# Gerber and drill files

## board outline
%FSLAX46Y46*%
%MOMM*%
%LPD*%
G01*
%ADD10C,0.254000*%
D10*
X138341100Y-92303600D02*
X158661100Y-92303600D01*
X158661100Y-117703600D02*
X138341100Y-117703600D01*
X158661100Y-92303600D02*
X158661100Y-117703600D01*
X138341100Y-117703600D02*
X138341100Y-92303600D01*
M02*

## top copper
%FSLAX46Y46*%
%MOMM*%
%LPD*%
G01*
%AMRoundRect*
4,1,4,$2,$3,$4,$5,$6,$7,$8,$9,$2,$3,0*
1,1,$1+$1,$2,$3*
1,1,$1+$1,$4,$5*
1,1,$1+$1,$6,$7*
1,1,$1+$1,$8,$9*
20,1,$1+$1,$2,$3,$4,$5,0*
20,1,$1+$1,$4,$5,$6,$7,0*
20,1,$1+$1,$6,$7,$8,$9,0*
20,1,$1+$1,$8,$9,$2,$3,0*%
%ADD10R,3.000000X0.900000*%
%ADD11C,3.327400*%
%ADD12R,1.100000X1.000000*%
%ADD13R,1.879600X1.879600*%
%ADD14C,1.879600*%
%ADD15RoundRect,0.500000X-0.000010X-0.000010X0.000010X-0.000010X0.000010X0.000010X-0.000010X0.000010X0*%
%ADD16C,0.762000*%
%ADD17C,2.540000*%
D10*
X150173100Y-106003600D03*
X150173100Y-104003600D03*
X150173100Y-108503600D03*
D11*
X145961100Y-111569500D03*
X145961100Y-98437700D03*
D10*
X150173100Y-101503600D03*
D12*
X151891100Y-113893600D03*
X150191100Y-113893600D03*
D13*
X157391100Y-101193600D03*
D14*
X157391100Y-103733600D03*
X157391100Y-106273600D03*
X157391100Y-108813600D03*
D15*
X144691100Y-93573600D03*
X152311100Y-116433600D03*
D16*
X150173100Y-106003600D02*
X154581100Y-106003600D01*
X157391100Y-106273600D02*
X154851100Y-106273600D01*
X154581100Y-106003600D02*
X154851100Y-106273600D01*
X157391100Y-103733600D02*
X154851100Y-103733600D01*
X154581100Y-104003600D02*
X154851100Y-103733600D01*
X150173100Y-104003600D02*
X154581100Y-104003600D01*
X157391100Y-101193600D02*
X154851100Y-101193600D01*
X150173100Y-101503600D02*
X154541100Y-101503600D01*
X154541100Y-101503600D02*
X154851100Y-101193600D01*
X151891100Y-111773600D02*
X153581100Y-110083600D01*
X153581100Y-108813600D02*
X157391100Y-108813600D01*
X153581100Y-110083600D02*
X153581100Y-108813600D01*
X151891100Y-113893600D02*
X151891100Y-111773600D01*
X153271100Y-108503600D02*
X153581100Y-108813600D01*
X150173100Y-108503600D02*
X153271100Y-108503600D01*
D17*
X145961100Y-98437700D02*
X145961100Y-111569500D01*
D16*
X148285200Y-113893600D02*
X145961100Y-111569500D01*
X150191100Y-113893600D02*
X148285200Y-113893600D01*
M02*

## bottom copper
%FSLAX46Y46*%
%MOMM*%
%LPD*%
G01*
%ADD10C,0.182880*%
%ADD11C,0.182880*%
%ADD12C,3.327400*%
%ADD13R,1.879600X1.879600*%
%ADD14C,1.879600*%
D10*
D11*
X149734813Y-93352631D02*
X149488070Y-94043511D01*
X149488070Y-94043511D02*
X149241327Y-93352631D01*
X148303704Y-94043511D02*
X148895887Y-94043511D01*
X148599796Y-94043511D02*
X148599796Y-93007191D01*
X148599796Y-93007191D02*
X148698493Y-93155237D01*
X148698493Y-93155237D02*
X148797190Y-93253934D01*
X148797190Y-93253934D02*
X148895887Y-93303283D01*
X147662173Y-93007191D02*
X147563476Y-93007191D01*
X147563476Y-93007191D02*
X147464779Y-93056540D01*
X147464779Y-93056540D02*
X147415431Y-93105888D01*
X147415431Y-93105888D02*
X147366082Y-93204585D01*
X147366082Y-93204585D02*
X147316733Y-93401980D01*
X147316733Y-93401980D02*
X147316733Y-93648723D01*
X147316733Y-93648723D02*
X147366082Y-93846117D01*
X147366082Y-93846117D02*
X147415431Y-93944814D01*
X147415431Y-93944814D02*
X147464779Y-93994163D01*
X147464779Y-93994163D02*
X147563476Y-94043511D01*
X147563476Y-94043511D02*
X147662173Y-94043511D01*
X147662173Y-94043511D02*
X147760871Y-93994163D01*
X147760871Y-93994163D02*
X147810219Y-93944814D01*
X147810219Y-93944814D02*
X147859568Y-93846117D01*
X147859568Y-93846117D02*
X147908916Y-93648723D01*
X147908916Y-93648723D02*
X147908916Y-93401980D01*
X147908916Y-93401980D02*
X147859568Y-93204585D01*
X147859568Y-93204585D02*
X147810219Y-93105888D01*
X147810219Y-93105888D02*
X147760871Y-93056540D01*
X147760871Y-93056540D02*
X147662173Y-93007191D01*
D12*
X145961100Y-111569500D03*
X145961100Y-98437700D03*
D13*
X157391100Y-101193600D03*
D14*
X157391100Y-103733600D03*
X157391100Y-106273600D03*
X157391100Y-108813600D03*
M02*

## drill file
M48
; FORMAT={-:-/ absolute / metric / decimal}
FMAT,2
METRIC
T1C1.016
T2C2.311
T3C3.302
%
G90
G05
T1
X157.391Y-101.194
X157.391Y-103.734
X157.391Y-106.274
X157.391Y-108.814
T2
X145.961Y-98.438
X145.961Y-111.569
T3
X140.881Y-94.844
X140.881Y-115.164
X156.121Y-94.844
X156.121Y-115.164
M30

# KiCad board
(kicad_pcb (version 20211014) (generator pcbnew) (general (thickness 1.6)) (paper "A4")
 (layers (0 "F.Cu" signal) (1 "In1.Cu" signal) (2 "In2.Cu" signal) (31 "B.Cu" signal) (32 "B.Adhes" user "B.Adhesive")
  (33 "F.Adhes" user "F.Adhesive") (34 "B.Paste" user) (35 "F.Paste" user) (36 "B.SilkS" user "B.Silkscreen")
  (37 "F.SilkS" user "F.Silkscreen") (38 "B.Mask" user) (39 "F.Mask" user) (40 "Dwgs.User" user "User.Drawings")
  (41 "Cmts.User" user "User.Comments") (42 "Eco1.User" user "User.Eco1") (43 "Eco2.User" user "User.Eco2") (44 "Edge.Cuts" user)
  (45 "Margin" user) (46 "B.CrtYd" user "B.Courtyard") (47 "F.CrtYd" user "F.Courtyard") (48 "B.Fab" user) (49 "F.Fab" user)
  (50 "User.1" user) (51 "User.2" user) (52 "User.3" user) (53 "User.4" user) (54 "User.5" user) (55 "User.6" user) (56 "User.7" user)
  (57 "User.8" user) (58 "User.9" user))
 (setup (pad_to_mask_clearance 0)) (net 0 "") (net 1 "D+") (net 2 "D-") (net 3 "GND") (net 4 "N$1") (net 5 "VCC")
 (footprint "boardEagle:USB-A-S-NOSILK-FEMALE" (layer "F.Cu") (at 145.9611 105.0036)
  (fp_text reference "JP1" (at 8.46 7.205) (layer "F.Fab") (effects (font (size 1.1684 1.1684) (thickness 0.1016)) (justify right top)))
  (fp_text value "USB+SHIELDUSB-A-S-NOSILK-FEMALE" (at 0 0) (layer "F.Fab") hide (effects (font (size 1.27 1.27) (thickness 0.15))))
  (pad "D+" smd rect (at 4.212 1) (size 3 0.9) (layers "F.Cu" "F.Paste" "F.Mask") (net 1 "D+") (solder_mask_margin 0.1016))
  (pad "D-" smd rect (at 4.212 -1) (size 3 0.9) (layers "F.Cu" "F.Paste" "F.Mask") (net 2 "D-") (solder_mask_margin 0.1016))
  (pad "GND" smd rect (at 4.212 3.5) (size 3 0.9) (layers "F.Cu" "F.Paste" "F.Mask") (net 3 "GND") (solder_mask_margin 0.1016))
  (pad "S1" thru_hole circle (at 0 6.5659 270) (size 3.3274 3.3274) (drill 2.3114) (layers *.Cu *.Mask) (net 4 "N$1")
   (solder_mask_margin 0.1016))
  (pad "S2" thru_hole circle (at 0 -6.5659 270) (size 3.3274 3.3274) (drill 2.3114) (layers *.Cu *.Mask) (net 4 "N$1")
   (solder_mask_margin 0.1016))
  (pad "VBUS" smd rect (at 4.212 -3.5) (size 3 0.9) (layers "F.Cu" "F.Paste" "F.Mask") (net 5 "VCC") (solder_mask_margin 0.1016)))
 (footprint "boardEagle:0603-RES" (layer "F.Cu") (at 151.0411 113.8936 180)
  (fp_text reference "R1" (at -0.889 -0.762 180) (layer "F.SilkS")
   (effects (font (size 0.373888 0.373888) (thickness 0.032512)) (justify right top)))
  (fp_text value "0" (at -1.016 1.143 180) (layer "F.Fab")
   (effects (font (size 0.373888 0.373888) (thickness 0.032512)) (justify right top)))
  (pad "1" smd rect (at -0.85 0 180) (size 1.1 1) (layers "F.Cu" "F.Paste" "F.Mask") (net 3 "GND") (solder_mask_margin 0.1016))
  (pad "2" smd rect (at 0.85 0 180) (size 1.1 1) (layers "F.Cu" "F.Paste" "F.Mask") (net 4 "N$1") (solder_mask_margin 0.1016)))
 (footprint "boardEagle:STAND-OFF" (layer "F.Cu") (at 140.8811 94.8436)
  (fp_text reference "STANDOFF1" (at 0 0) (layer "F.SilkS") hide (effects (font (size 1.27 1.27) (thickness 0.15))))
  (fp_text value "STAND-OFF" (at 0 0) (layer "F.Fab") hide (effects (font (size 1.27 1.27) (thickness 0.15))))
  (pad "" np_thru_hole circle (at 0 0) (size 3.302 3.302) (drill 3.302) (layers *.Cu *.Mask)))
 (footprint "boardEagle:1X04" (layer "F.Cu") (at 157.3911 101.1936 -90)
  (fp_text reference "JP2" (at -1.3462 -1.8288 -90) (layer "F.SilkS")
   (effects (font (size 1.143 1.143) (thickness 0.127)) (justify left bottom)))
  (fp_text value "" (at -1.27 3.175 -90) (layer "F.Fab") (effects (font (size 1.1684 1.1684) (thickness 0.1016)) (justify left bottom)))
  (pad "1" thru_hole rect (at 0 0) (size 1.8796 1.8796) (drill 1.016) (layers *.Cu *.Mask) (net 5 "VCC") (solder_mask_margin 0.1016))
  (pad "2" thru_hole circle (at 2.54 0) (size 1.8796 1.8796) (drill 1.016) (layers *.Cu *.Mask) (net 2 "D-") (solder_mask_margin 0.1016))
  (pad "3" thru_hole circle (at 5.08 0) (size 1.8796 1.8796) (drill 1.016) (layers *.Cu *.Mask) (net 1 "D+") (solder_mask_margin 0.1016))
  (pad "4" thru_hole circle (at 7.62 0) (size 1.8796 1.8796) (drill 1.016) (layers *.Cu *.Mask) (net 3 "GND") (solder_mask_margin 0.1016)))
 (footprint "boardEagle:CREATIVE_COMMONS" (layer "F.Cu") (at 123.1011 135.4836)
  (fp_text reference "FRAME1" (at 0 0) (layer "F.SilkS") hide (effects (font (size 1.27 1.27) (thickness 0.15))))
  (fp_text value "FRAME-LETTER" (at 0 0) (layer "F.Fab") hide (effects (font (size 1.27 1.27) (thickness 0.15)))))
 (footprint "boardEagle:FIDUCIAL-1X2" (layer "F.Cu") (at 144.6911 93.5736)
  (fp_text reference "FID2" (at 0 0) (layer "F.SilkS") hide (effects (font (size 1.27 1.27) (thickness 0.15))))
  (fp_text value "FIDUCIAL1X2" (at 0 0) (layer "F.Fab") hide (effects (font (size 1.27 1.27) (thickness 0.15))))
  (pad "1" smd roundrect (at 0 0) (size 1 1) (layers "F.Cu" "F.Mask") (roundrect_rratio 0.5) (solder_mask_margin 0.1016)))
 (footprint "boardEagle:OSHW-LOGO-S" (layer "F.Cu") (at 147.8661 115.1636 90)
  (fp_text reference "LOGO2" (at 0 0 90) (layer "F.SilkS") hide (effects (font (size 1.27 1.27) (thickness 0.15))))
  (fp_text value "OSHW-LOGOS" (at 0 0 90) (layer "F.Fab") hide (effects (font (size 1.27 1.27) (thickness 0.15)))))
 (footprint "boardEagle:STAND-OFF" (layer "F.Cu") (at 156.1211 115.1636)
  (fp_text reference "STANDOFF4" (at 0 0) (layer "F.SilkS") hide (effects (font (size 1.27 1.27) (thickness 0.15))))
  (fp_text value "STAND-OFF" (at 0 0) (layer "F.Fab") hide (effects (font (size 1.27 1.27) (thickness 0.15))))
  (pad "" np_thru_hole circle (at 0 0) (size 3.302 3.302) (drill 3.302) (layers *.Cu *.Mask)))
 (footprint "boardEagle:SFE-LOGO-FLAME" (layer "F.Cu") (at 149.1361 96.1136 90)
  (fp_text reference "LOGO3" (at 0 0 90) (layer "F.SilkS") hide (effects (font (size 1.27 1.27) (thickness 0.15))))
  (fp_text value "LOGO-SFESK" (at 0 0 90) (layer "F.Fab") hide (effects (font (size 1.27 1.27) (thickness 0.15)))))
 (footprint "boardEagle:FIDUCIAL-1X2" (layer "F.Cu") (at 152.3111 116.4336)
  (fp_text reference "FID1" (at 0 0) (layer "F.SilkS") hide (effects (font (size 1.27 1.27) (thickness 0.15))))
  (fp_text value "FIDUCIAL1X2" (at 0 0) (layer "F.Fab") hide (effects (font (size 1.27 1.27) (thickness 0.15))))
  (pad "1" smd roundrect (at 0 0) (size 1 1) (layers "F.Cu" "F.Mask") (roundrect_rratio 0.5) (solder_mask_margin 0.1016)))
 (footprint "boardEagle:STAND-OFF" (layer "F.Cu") (at 140.8811 115.1636)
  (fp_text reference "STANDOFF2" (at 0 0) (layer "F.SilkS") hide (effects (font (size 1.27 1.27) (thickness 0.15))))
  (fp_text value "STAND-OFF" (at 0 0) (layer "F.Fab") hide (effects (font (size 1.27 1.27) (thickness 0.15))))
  (pad "" np_thru_hole circle (at 0 0) (size 3.302 3.302) (drill 3.302) (layers *.Cu *.Mask)))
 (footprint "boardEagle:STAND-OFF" (layer "F.Cu") (at 156.1211 94.8436)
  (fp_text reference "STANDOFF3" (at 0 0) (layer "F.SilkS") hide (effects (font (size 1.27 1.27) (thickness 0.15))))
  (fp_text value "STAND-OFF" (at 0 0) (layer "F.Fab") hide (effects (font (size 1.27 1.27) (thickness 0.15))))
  (pad "" np_thru_hole circle (at 0 0) (size 3.302 3.302) (drill 3.302) (layers *.Cu *.Mask)))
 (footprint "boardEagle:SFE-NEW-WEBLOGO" (layer "B.Cu") (at 151.0411 95.8596 -90)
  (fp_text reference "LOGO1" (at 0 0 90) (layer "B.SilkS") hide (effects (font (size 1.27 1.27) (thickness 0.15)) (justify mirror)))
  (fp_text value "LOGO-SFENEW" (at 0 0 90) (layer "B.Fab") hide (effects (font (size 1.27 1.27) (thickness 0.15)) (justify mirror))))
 (gr_line (start 138.3411 92.3036) (end 158.6611 92.3036) (layer "Edge.Cuts") (width 0.254))
 (gr_line (start 158.6611 117.7036) (end 138.3411 117.7036) (layer "Edge.Cuts") (width 0.254))
 (gr_line (start 158.6611 92.3036) (end 158.6611 117.7036) (layer "Edge.Cuts") (width 0.254))
 (gr_line (start 138.3411 117.7036) (end 138.3411 92.3036) (layer "Edge.Cuts") (width 0.254))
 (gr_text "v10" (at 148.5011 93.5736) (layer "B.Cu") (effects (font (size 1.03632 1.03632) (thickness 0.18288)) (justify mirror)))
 (segment (start 150.1731 106.0036) (end 154.5811 106.0036) (width 0.762) (layer "F.Cu") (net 1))
 (segment (start 157.3911 106.2736) (end 154.8511 106.2736) (width 0.762) (layer "F.Cu") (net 1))
 (segment (start 154.5811 106.0036) (end 154.8511 106.2736) (width 0.762) (layer "F.Cu") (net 1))
 (segment (start 157.3911 103.7336) (end 154.8511 103.7336) (width 0.762) (layer "F.Cu") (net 2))
 (segment (start 154.5811 104.0036) (end 154.8511 103.7336) (width 0.762) (layer "F.Cu") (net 2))
 (segment (start 150.1731 104.0036) (end 154.5811 104.0036) (width 0.762) (layer "F.Cu") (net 2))
 (segment (start 157.3911 101.1936) (end 154.8511 101.1936) (width 0.762) (layer "F.Cu") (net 5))
 (segment (start 150.1731 101.5036) (end 154.5411 101.5036) (width 0.762) (layer "F.Cu") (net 5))
 (segment (start 154.5411 101.5036) (end 154.8511 101.1936) (width 0.762) (layer "F.Cu") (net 5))
 (segment (start 151.8911 111.7736) (end 153.5811 110.0836) (width 0.762) (layer "F.Cu") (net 3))
 (segment (start 153.5811 108.8136) (end 157.3911 108.8136) (width 0.762) (layer "F.Cu") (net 3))
 (segment (start 153.5811 110.0836) (end 153.5811 108.8136) (width 0.762) (layer "F.Cu") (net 3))
 (segment (start 151.8911 113.8936) (end 151.8911 111.7736) (width 0.762) (layer "F.Cu") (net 3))
 (segment (start 153.2711 108.5036) (end 153.5811 108.8136) (width 0.762) (layer "F.Cu") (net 3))
 (segment (start 150.1731 108.5036) (end 153.2711 108.5036) (width 0.762) (layer "F.Cu") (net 3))
 (segment (start 145.9611 98.4377) (end 145.9611 111.5695) (width 2.54) (layer "F.Cu") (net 4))
 (segment (start 148.2852 113.8936) (end 145.9611 111.5695) (width 0.762) (layer "F.Cu") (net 4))
 (segment (start 150.1911 113.8936) (end 148.2852 113.8936) (width 0.762) (layer "F.Cu") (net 4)))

